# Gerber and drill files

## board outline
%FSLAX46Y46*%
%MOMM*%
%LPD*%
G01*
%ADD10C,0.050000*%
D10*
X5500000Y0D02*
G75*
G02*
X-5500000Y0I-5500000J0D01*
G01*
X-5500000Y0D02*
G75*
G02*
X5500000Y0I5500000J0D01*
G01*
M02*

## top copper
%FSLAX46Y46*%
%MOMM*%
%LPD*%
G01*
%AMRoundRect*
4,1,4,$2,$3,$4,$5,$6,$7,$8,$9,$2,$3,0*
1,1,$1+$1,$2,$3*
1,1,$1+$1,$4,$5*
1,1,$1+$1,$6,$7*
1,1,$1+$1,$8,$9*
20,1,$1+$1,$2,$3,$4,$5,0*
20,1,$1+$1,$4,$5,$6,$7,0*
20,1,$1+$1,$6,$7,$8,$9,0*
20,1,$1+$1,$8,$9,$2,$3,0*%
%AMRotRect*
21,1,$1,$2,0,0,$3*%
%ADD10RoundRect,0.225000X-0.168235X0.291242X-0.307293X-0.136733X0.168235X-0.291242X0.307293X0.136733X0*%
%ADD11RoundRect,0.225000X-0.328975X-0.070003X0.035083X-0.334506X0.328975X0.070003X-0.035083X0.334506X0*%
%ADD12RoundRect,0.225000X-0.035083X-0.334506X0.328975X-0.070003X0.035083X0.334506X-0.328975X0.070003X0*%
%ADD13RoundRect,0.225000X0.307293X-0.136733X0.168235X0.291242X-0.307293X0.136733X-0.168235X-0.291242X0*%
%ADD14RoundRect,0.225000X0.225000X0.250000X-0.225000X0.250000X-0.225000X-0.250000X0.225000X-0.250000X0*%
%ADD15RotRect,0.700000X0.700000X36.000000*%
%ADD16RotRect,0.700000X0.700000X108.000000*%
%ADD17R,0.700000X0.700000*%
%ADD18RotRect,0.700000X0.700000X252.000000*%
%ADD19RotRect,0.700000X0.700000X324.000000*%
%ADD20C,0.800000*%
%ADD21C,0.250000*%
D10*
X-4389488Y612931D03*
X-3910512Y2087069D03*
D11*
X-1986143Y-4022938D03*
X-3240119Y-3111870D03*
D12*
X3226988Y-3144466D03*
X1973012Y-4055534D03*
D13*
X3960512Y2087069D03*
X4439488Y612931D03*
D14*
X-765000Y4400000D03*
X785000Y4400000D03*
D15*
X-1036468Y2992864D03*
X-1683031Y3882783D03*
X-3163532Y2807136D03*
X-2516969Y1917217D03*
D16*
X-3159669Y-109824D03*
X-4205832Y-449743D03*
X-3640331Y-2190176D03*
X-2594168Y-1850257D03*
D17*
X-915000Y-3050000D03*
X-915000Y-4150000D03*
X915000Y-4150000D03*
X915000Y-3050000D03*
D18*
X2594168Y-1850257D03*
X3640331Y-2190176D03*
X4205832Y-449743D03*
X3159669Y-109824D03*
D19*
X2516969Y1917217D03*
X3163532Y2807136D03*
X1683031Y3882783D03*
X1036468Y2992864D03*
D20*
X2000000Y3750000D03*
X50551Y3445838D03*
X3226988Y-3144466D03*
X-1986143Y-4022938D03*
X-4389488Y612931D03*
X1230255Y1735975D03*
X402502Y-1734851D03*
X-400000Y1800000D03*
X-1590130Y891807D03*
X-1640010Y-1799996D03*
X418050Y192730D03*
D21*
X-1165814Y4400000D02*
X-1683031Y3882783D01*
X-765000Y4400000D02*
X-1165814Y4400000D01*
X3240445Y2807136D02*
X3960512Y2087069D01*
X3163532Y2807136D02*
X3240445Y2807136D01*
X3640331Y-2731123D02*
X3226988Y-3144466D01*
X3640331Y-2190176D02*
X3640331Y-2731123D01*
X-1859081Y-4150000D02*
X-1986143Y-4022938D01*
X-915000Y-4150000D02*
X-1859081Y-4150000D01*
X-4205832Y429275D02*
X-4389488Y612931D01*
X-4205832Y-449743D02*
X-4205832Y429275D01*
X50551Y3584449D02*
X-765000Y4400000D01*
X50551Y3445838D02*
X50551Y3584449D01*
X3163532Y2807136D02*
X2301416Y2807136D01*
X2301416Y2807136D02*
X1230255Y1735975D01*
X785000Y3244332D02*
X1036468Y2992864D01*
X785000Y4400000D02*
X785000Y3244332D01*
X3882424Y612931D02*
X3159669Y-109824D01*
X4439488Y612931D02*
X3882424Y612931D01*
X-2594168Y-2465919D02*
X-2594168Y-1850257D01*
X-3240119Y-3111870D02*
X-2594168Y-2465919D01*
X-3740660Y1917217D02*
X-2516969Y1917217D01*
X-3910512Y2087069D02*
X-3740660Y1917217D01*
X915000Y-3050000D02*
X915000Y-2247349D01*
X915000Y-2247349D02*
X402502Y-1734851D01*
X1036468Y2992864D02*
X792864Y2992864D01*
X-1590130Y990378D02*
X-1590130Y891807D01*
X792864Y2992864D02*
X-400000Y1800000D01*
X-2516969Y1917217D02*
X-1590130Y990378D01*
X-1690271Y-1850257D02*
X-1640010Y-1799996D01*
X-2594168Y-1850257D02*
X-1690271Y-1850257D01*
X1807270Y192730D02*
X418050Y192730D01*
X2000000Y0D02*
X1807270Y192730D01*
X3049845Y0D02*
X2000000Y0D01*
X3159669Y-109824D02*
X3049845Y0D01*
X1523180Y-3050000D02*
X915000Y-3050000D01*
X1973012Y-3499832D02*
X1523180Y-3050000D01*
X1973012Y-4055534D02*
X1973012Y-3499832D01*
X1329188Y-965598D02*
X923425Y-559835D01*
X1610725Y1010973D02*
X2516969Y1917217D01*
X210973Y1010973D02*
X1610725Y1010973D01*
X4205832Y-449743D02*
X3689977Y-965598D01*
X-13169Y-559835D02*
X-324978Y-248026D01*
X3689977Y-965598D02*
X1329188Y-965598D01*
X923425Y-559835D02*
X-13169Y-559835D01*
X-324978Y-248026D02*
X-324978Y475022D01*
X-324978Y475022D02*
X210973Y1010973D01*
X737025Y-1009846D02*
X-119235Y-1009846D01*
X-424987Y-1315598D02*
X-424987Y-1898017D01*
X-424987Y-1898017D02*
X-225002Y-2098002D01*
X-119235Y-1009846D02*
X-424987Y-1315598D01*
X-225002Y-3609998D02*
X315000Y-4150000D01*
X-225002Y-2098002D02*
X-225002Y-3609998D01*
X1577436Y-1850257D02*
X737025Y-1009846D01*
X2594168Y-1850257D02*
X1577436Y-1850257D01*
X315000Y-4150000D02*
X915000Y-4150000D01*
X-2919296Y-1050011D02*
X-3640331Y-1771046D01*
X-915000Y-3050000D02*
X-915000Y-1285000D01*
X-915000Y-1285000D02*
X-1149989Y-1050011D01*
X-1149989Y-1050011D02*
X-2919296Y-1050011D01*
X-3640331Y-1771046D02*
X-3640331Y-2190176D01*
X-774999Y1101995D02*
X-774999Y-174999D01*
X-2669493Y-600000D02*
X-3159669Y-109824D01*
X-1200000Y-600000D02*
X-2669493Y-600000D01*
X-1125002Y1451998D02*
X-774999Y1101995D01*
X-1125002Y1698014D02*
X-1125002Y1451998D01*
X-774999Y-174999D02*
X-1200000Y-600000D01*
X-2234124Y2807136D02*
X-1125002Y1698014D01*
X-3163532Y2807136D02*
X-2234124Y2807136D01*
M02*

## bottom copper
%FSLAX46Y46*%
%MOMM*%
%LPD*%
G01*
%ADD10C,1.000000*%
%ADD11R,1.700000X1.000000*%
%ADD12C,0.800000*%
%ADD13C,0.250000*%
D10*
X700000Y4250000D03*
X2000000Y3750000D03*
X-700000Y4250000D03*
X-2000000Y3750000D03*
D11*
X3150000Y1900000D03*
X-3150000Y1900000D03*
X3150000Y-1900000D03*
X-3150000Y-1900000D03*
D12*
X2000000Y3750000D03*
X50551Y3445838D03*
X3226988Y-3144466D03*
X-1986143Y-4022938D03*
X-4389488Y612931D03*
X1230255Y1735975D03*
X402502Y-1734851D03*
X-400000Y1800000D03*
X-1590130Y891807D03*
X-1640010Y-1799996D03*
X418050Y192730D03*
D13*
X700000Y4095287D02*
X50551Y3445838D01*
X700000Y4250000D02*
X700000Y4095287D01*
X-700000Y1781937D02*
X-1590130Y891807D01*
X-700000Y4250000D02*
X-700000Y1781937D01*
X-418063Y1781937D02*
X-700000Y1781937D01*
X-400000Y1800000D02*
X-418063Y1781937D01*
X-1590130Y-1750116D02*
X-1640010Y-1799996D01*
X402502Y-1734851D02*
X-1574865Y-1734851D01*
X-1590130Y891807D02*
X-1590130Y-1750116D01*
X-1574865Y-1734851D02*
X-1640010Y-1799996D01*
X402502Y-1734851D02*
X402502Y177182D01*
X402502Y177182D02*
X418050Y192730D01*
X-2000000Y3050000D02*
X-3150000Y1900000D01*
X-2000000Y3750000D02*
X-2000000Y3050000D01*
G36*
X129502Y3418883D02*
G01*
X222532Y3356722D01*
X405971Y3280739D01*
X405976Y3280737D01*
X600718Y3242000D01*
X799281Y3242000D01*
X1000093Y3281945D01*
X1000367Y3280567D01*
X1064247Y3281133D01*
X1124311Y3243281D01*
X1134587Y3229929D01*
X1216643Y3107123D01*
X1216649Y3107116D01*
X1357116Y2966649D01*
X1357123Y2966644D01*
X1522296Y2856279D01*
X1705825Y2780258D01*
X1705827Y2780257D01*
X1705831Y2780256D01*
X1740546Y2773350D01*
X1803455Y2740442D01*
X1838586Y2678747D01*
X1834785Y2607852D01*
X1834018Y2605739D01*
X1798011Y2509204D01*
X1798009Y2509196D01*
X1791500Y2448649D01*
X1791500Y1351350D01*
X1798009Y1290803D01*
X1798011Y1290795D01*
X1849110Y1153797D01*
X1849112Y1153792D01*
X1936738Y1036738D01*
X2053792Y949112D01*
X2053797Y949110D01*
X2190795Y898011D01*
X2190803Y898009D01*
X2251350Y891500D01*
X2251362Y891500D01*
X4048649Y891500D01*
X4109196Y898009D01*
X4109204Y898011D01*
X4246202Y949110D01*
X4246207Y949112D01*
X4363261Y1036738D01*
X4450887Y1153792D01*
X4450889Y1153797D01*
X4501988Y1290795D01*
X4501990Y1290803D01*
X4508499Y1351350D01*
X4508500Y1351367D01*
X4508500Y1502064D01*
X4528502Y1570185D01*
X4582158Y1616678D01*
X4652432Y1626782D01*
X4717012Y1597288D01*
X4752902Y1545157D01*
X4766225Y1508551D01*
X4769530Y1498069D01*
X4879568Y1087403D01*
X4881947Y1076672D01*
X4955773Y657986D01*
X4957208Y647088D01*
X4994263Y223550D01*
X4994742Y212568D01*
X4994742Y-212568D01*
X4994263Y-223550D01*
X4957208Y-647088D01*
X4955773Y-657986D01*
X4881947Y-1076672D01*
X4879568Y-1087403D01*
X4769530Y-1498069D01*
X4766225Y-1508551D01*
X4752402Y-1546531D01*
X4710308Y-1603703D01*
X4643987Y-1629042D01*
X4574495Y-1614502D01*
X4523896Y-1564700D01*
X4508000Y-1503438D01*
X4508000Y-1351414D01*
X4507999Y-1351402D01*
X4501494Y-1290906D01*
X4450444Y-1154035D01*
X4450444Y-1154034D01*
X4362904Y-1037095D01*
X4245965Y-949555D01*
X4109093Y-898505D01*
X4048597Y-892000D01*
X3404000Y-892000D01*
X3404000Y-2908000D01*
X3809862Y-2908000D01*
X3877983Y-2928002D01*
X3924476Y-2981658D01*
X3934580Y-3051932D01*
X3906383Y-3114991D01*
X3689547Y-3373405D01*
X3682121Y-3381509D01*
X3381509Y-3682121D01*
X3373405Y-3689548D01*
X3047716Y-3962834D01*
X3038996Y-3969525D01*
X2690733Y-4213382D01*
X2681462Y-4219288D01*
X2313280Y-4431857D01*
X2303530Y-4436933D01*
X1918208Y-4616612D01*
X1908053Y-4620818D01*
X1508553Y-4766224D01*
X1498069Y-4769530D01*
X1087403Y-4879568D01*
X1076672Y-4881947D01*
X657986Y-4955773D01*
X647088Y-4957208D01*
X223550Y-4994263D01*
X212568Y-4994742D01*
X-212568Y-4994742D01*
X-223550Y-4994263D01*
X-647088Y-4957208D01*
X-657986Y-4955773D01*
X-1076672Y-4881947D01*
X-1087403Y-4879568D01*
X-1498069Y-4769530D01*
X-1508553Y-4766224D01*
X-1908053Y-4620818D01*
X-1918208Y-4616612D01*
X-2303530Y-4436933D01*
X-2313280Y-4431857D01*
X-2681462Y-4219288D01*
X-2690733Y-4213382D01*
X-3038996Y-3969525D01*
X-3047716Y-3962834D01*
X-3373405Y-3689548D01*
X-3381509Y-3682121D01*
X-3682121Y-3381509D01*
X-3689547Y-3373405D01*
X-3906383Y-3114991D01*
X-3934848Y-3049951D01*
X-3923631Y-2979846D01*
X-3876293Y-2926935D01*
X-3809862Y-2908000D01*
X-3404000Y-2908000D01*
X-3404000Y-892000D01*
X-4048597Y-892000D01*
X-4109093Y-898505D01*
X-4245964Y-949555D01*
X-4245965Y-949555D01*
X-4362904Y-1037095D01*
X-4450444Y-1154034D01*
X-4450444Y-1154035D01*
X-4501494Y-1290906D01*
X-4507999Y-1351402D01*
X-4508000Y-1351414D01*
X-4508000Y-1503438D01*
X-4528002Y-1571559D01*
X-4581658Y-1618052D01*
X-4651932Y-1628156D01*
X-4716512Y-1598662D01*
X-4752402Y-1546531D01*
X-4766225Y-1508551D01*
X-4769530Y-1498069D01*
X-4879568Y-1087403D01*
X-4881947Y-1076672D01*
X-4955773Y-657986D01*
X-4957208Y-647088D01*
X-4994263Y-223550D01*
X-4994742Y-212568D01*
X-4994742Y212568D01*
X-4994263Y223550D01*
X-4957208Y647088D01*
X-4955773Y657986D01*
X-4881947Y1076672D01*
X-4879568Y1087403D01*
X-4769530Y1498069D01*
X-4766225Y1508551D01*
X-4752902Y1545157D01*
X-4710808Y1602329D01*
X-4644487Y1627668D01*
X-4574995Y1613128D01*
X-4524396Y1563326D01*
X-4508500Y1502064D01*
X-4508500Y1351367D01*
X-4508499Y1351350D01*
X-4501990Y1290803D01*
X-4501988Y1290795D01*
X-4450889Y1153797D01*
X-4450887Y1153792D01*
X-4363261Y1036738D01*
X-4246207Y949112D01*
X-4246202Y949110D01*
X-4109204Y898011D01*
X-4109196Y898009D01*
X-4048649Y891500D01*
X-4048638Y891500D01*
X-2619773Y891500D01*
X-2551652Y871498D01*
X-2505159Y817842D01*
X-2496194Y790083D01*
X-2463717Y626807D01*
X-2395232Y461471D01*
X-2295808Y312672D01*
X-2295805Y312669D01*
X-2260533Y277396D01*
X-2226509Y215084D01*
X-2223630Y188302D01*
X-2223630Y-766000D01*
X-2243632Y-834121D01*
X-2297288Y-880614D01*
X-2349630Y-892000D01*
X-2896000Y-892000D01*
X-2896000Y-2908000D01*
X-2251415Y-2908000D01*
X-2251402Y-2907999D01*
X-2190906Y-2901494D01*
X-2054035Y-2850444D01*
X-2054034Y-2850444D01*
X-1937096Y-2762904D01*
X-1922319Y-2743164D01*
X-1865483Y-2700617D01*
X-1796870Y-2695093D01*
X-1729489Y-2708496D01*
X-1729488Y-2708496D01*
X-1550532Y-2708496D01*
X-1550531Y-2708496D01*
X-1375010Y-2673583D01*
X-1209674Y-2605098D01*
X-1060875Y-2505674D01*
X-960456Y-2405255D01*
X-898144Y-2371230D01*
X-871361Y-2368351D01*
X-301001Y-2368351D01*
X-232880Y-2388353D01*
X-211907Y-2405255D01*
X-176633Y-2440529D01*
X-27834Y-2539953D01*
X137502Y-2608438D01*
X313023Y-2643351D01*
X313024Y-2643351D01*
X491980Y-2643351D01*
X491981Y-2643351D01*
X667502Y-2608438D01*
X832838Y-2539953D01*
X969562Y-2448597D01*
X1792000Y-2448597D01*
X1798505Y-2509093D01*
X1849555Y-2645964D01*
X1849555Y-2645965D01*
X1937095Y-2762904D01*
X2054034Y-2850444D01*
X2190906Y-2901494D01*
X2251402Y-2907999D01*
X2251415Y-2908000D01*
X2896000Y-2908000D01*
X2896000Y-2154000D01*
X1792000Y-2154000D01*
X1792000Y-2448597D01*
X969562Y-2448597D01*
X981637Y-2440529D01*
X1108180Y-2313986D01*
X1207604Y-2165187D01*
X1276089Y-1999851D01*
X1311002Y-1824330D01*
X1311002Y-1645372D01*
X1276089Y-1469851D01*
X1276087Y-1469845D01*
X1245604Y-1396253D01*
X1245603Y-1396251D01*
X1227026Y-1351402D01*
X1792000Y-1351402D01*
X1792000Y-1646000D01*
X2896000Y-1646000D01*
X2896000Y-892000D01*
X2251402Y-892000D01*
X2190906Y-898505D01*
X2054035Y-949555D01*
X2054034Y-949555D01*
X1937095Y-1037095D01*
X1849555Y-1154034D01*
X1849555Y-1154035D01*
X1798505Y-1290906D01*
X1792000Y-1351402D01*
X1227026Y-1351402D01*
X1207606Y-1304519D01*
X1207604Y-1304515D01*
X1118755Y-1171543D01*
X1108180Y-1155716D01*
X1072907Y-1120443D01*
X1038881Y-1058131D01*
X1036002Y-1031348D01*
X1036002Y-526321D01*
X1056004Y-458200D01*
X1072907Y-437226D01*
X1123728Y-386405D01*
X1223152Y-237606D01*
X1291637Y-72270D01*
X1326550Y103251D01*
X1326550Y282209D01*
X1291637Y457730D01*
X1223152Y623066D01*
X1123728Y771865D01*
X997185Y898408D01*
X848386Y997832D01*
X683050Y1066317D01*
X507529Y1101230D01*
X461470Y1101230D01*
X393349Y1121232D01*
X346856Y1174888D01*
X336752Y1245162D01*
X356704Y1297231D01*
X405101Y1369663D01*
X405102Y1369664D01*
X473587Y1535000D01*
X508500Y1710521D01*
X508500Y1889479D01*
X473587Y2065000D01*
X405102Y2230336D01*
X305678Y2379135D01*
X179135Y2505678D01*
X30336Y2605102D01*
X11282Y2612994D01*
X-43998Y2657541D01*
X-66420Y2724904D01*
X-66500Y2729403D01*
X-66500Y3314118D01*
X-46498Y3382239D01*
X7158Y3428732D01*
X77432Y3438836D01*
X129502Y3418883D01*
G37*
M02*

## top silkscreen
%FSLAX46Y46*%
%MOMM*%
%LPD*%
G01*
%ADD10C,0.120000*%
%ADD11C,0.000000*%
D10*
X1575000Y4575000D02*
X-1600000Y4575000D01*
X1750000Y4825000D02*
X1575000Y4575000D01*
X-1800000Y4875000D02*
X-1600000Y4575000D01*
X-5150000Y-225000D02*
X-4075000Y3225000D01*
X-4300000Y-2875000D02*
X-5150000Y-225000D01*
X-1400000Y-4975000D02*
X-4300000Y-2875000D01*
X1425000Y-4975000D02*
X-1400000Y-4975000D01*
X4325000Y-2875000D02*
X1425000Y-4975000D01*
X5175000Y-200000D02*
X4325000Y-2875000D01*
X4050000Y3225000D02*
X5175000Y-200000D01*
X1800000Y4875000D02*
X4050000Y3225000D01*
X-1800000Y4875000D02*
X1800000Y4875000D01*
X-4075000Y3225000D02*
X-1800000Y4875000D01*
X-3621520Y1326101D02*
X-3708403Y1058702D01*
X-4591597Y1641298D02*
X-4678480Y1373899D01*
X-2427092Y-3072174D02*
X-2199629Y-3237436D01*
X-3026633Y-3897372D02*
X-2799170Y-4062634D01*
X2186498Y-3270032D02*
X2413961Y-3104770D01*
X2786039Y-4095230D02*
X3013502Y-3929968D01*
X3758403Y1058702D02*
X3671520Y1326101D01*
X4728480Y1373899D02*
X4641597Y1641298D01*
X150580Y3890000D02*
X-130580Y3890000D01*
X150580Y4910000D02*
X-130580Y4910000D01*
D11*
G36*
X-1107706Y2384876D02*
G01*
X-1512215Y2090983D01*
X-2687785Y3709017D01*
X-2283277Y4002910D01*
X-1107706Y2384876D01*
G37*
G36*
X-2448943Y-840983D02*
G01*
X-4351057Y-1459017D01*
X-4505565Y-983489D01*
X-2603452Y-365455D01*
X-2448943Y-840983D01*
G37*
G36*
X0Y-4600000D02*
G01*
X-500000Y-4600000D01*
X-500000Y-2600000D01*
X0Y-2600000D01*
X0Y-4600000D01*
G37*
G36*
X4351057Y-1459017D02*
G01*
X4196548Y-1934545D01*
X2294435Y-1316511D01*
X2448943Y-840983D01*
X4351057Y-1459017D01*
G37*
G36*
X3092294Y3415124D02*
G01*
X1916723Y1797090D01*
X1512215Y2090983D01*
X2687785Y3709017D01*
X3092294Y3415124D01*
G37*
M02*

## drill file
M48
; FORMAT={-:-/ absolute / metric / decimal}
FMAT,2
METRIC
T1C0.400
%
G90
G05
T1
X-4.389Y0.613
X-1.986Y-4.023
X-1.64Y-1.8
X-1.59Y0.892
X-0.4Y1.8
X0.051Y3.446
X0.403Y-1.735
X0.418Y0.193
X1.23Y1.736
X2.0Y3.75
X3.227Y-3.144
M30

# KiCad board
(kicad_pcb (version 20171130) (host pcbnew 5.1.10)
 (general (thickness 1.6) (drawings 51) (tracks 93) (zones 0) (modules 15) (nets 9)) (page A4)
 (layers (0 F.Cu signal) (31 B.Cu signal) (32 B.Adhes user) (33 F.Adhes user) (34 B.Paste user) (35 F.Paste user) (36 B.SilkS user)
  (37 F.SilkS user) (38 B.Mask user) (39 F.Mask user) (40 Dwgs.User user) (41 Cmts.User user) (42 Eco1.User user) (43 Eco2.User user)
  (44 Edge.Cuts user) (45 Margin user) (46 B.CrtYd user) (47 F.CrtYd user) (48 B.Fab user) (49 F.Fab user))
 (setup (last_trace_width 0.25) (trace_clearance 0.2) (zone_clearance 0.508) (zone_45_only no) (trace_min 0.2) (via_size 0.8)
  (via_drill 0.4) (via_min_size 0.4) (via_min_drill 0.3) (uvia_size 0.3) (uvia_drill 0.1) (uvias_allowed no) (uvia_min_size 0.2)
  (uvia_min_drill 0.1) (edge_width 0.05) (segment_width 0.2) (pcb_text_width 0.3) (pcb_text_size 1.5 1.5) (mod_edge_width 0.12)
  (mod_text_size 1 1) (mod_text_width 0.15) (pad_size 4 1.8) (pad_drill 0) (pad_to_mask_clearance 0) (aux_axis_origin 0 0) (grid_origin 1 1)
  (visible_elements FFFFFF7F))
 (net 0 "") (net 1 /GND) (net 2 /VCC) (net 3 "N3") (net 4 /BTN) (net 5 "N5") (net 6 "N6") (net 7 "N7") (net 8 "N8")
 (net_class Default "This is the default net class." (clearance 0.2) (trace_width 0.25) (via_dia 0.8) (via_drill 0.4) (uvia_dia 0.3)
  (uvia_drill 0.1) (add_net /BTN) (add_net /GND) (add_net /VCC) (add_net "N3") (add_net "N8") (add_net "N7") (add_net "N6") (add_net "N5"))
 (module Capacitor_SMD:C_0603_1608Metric (layer F.Cu) (at -4.15 -1.35 252)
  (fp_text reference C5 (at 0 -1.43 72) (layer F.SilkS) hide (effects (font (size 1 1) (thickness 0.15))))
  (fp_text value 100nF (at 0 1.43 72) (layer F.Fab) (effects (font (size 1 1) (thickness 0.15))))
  (fp_line (start -0.14058 -0.51) (end 0.14058 -0.51) (layer F.SilkS) (width 0.12))
  (fp_line (start -0.14058 0.51) (end 0.14058 0.51) (layer F.SilkS) (width 0.12))
  (pad 2 smd roundrect (at 0.775 0 252) (size 0.9 0.95) (layers F.Cu F.Paste F.Mask) (roundrect_rratio 0.25) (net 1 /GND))
  (pad 1 smd roundrect (at -0.775 0 252) (size 0.9 0.95) (layers F.Cu F.Paste F.Mask) (roundrect_rratio 0.25) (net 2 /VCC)))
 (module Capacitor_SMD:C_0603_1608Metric (layer F.Cu) (at -2.613131 3.567404 324)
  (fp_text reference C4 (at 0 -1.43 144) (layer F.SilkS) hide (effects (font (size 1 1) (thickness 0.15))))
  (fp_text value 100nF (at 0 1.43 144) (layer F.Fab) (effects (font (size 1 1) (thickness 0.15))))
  (fp_line (start -0.14058 -0.51) (end 0.14058 -0.51) (layer F.SilkS) (width 0.12))
  (fp_line (start -0.14058 0.51) (end 0.14058 0.51) (layer F.SilkS) (width 0.12))
  (pad 2 smd roundrect (at 0.775 0 324) (size 0.9 0.95) (layers F.Cu F.Paste F.Mask) (roundrect_rratio 0.25) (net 1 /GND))
  (pad 1 smd roundrect (at -0.775 0 324) (size 0.9 0.95) (layers F.Cu F.Paste F.Mask) (roundrect_rratio 0.25) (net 2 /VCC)))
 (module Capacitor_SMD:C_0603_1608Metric (layer F.Cu) (at 2.6 3.6 36)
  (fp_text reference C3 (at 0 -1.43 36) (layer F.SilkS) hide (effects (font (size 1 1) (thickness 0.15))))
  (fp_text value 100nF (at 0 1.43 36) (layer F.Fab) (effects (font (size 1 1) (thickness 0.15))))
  (fp_line (start -0.14058 -0.51) (end 0.14058 -0.51) (layer F.SilkS) (width 0.12))
  (fp_line (start -0.14058 0.51) (end 0.14058 0.51) (layer F.SilkS) (width 0.12))
  (pad 2 smd roundrect (at 0.775 0 36) (size 0.9 0.95) (layers F.Cu F.Paste F.Mask) (roundrect_rratio 0.25) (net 1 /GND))
  (pad 1 smd roundrect (at -0.775 0 36) (size 0.9 0.95) (layers F.Cu F.Paste F.Mask) (roundrect_rratio 0.25) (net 2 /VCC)))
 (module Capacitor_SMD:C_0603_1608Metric (layer F.Cu) (at 4.2 -1.35 108)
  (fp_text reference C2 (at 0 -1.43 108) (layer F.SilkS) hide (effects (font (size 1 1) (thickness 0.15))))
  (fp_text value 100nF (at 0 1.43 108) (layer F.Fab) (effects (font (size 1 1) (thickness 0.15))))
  (fp_line (start -0.14058 -0.51) (end 0.14058 -0.51) (layer F.SilkS) (width 0.12))
  (fp_line (start -0.14058 0.51) (end 0.14058 0.51) (layer F.SilkS) (width 0.12))
  (pad 2 smd roundrect (at 0.775 0 108) (size 0.9 0.95) (layers F.Cu F.Paste F.Mask) (roundrect_rratio 0.25) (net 1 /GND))
  (pad 1 smd roundrect (at -0.775 0 108) (size 0.9 0.95) (layers F.Cu F.Paste F.Mask) (roundrect_rratio 0.25) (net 2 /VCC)))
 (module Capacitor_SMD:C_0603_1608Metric (layer F.Cu) (at 0.01 -4.4 180)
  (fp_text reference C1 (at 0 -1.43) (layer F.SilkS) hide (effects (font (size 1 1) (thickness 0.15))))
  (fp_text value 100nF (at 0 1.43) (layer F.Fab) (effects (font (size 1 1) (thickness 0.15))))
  (fp_line (start -0.14058 -0.51) (end 0.14058 -0.51) (layer F.SilkS) (width 0.12))
  (fp_line (start -0.14058 0.51) (end 0.14058 0.51) (layer F.SilkS) (width 0.12))
  (pad 2 smd roundrect (at 0.775 0 180) (size 0.9 0.95) (layers F.Cu F.Paste F.Mask) (roundrect_rratio 0.25) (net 1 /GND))
  (pad 1 smd roundrect (at -0.775 0 180) (size 0.9 0.95) (layers F.Cu F.Paste F.Mask) (roundrect_rratio 0.25) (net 2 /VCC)))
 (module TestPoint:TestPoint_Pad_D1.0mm (layer B.Cu) (at 0.7 -4.25)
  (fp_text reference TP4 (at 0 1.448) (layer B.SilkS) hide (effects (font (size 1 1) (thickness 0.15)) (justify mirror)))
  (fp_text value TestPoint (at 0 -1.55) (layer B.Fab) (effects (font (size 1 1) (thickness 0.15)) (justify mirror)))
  (pad 1 smd circle (at 0 0) (size 1 1) (layers B.Cu B.Mask) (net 1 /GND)))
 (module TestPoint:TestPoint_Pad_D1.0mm (layer B.Cu) (at 2 -3.75)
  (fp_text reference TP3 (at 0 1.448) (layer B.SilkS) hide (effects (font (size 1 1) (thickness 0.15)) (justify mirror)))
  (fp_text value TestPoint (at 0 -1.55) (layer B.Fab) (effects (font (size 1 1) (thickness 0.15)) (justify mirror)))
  (pad 1 smd circle (at 0 0) (size 1 1) (layers B.Cu B.Mask) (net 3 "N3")))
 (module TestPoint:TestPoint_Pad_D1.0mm (layer B.Cu) (at -0.7 -4.25)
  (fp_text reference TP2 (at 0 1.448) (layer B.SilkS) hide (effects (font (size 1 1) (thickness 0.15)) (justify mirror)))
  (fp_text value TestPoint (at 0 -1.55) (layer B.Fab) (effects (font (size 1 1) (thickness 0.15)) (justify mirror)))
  (pad 1 smd circle (at 0 0) (size 1 1) (layers B.Cu B.Mask) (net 2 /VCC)))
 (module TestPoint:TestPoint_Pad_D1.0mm (layer B.Cu) (at -2 -3.75)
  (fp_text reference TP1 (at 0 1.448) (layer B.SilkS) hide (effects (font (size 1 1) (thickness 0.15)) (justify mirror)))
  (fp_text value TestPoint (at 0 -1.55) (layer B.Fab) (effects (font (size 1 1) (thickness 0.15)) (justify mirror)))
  (pad 1 smd circle (at 0 0) (size 1 1) (layers B.Cu B.Mask) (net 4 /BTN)))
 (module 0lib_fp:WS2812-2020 (layer F.Cu) (at -2.1 -2.9 36)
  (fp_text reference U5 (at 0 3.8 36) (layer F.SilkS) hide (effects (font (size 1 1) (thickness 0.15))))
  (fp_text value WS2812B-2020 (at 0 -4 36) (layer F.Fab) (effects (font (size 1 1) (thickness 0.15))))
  (fp_poly (pts (xy 0 -1) (xy 0.5 -1) (xy 0.5 1) (xy 0 1)) (layer F.SilkS) (width 0))
  (pad 1 smd rect (at 0.915 0.55 36) (size 0.7 0.7) (layers F.Cu F.Paste F.Mask))
  (pad 2 smd rect (at 0.915 -0.55 36) (size 0.7 0.7) (layers F.Cu F.Paste F.Mask) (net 1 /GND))
  (pad 3 smd rect (at -0.915 -0.55 36) (size 0.7 0.7) (layers F.Cu F.Paste F.Mask) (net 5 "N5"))
  (pad 4 smd rect (at -0.915 0.55 36) (size 0.7 0.7) (layers F.Cu F.Paste F.Mask) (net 2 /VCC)))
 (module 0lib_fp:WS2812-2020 (layer F.Cu) (at -3.4 1.15 108)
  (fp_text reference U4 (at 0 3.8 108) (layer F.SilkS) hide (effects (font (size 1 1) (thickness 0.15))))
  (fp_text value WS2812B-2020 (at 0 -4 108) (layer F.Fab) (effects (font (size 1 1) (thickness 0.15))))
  (fp_poly (pts (xy 0 -1) (xy 0.5 -1) (xy 0.5 1) (xy 0 1)) (layer F.SilkS) (width 0))
  (pad 1 smd rect (at 0.915 0.55 108) (size 0.7 0.7) (layers F.Cu F.Paste F.Mask) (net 5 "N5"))
  (pad 2 smd rect (at 0.915 -0.55 108) (size 0.7 0.7) (layers F.Cu F.Paste F.Mask) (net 1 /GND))
  (pad 3 smd rect (at -0.915 -0.55 108) (size 0.7 0.7) (layers F.Cu F.Paste F.Mask) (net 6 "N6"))
  (pad 4 smd rect (at -0.915 0.55 108) (size 0.7 0.7) (layers F.Cu F.Paste F.Mask) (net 2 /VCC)))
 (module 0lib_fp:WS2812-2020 (layer F.Cu) (at 0 3.6 180)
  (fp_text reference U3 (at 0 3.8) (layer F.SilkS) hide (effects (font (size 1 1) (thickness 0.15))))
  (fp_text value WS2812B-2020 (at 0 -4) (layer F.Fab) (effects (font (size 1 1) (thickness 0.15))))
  (fp_poly (pts (xy 0 -1) (xy 0.5 -1) (xy 0.5 1) (xy 0 1)) (layer F.SilkS) (width 0))
  (pad 1 smd rect (at 0.915 0.55 180) (size 0.7 0.7) (layers F.Cu F.Paste F.Mask) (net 6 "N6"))
  (pad 2 smd rect (at 0.915 -0.55 180) (size 0.7 0.7) (layers F.Cu F.Paste F.Mask) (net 1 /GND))
  (pad 3 smd rect (at -0.915 -0.55 180) (size 0.7 0.7) (layers F.Cu F.Paste F.Mask) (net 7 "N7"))
  (pad 4 smd rect (at -0.915 0.55 180) (size 0.7 0.7) (layers F.Cu F.Paste F.Mask) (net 2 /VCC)))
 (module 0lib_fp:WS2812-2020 (layer F.Cu) (at 3.4 1.15 252)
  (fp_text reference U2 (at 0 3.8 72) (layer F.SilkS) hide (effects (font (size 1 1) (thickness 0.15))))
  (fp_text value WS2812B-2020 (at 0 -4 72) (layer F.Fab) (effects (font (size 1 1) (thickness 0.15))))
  (fp_poly (pts (xy 0 -1) (xy 0.5 -1) (xy 0.5 1) (xy 0 1)) (layer F.SilkS) (width 0))
  (pad 1 smd rect (at 0.915 0.55 252) (size 0.7 0.7) (layers F.Cu F.Paste F.Mask) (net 7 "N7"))
  (pad 2 smd rect (at 0.915 -0.55 252) (size 0.7 0.7) (layers F.Cu F.Paste F.Mask) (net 1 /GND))
  (pad 3 smd rect (at -0.915 -0.55 252) (size 0.7 0.7) (layers F.Cu F.Paste F.Mask) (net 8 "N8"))
  (pad 4 smd rect (at -0.915 0.55 252) (size 0.7 0.7) (layers F.Cu F.Paste F.Mask) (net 2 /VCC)))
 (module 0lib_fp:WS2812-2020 (layer F.Cu) (at 2.1 -2.9 324)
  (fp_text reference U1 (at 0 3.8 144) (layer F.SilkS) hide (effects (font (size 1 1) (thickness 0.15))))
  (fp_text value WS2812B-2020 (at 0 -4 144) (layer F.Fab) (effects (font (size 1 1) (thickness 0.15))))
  (fp_poly (pts (xy 0 -1) (xy 0.5 -1) (xy 0.5 1) (xy 0 1)) (layer F.SilkS) (width 0))
  (pad 1 smd rect (at 0.915 0.55 324) (size 0.7 0.7) (layers F.Cu F.Paste F.Mask) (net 8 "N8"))
  (pad 2 smd rect (at 0.915 -0.55 324) (size 0.7 0.7) (layers F.Cu F.Paste F.Mask) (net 1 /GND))
  (pad 3 smd rect (at -0.915 -0.55 324) (size 0.7 0.7) (layers F.Cu F.Paste F.Mask) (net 3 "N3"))
  (pad 4 smd rect (at -0.915 0.55 324) (size 0.7 0.7) (layers F.Cu F.Paste F.Mask) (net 2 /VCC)))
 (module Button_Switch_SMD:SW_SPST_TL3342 (layer B.Cu) (at 0 0)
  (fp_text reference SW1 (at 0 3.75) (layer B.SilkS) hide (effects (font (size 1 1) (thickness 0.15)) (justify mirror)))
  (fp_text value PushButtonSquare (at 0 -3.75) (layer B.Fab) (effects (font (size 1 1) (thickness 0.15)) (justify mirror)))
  (pad 2 smd rect (at 3.15 -1.9) (size 1.7 1) (layers B.Cu B.Paste B.Mask) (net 4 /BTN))
  (pad 2 smd rect (at -3.15 -1.9) (size 1.7 1) (layers B.Cu B.Paste B.Mask) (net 4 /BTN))
  (pad 1 smd rect (at 3.15 1.9) (size 1.7 1) (layers B.Cu B.Paste B.Mask) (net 1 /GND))
  (pad 1 smd rect (at -3.15 1.9) (size 1.7 1) (layers B.Cu B.Paste B.Mask) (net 1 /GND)))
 (gr_line (start 1.575 -4.575) (end -1.6 -4.575) (layer F.SilkS) (width 0.12))
 (gr_line (start 1.75 -4.825) (end 1.575 -4.575) (layer F.SilkS) (width 0.12))
 (gr_line (start -1.8 -4.875) (end -1.6 -4.575) (layer F.SilkS) (width 0.12))
 (gr_line (start -5.15 0.225) (end -4.075 -3.225) (layer F.SilkS) (width 0.12))
 (gr_line (start -4.3 2.875) (end -5.15 0.225) (layer F.SilkS) (width 0.12))
 (gr_line (start -1.4 4.975) (end -4.3 2.875) (layer F.SilkS) (width 0.12))
 (gr_line (start 1.425 4.975) (end -1.4 4.975) (layer F.SilkS) (width 0.12))
 (gr_line (start 4.325 2.875) (end 1.425 4.975) (layer F.SilkS) (width 0.12))
 (gr_line (start 5.175 0.2) (end 4.325 2.875) (layer F.SilkS) (width 0.12))
 (gr_line (start 4.05 -3.225) (end 5.175 0.2) (layer F.SilkS) (width 0.12))
 (gr_line (start 1.8 -4.875) (end 4.05 -3.225) (layer F.SilkS) (width 0.12))
 (gr_line (start -1.8 -4.875) (end 1.8 -4.875) (layer F.SilkS) (width 0.12))
 (gr_line (start -4.075 -3.225) (end -1.8 -4.875) (layer F.SilkS) (width 0.12))
 (gr_circle (center 0 0) (end 0 -5.5) (layer Edge.Cuts) (width 0.05))
 (via (at 2 -3.75) (size 0.8) (drill 0.4) (layers F.Cu B.Cu) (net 3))
 (segment (start -1.165814 -4.4) (end -1.683031 -3.882783) (width 0.25) (layer F.Cu) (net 1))
 (segment (start -0.765 -4.4) (end -1.165814 -4.4) (width 0.25) (layer F.Cu) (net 1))
 (segment (start 3.240445 -2.807136) (end 3.960512 -2.087069) (width 0.25) (layer F.Cu) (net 1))
 (segment (start 3.163532 -2.807136) (end 3.240445 -2.807136) (width 0.25) (layer F.Cu) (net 1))
 (segment (start 3.640331 2.731123) (end 3.226988 3.144466) (width 0.25) (layer F.Cu) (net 1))
 (segment (start 3.640331 2.190176) (end 3.640331 2.731123) (width 0.25) (layer F.Cu) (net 1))
 (segment (start -1.859081 4.15) (end -1.986143 4.022938) (width 0.25) (layer F.Cu) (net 1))
 (segment (start -0.915 4.15) (end -1.859081 4.15) (width 0.25) (layer F.Cu) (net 1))
 (segment (start -4.205832 -0.429275) (end -4.389488 -0.612931) (width 0.25) (layer F.Cu) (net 1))
 (segment (start -4.205832 0.449743) (end -4.205832 -0.429275) (width 0.25) (layer F.Cu) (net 1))
 (via (at 0.050551 -3.445838) (size 0.8) (drill 0.4) (layers F.Cu B.Cu) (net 1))
 (segment (start 0.7 -4.095287) (end 0.050551 -3.445838) (width 0.25) (layer B.Cu) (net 1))
 (segment (start 0.7 -4.25) (end 0.7 -4.095287) (width 0.25) (layer B.Cu) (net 1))
 (segment (start 0.050551 -3.584449) (end -0.765 -4.4) (width 0.25) (layer F.Cu) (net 1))
 (segment (start 0.050551 -3.445838) (end 0.050551 -3.584449) (width 0.25) (layer F.Cu) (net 1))
 (via (at 3.226988 3.144466) (size 0.8) (drill 0.4) (layers F.Cu B.Cu) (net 1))
 (via (at -1.986143 4.022938) (size 0.8) (drill 0.4) (layers F.Cu B.Cu) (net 1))
 (via (at -4.389488 -0.612931) (size 0.8) (drill 0.4) (layers F.Cu B.Cu) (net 1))
 (segment (start 3.163532 -2.807136) (end 2.301416 -2.807136) (width 0.25) (layer F.Cu) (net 1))
 (segment (start 2.301416 -2.807136) (end 1.230255 -1.735975) (width 0.25) (layer F.Cu) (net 1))
 (via (at 1.230255 -1.735975) (size 0.8) (drill 0.4) (layers F.Cu B.Cu) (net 1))
 (segment (start 0.785 -3.244332) (end 1.036468 -2.992864) (width 0.25) (layer F.Cu) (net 2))
 (segment (start 0.785 -4.4) (end 0.785 -3.244332) (width 0.25) (layer F.Cu) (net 2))
 (segment (start 3.882424 -0.612931) (end 3.159669 0.109824) (width 0.25) (layer F.Cu) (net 2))
 (segment (start 4.439488 -0.612931) (end 3.882424 -0.612931) (width 0.25) (layer F.Cu) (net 2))
 (segment (start -2.594168 2.465919) (end -2.594168 1.850257) (width 0.25) (layer F.Cu) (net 2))
 (segment (start -3.240119 3.11187) (end -2.594168 2.465919) (width 0.25) (layer F.Cu) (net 2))
 (segment (start -3.74066 -1.917217) (end -2.516969 -1.917217) (width 0.25) (layer F.Cu) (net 2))
 (segment (start -3.910512 -2.087069) (end -3.74066 -1.917217) (width 0.25) (layer F.Cu) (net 2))
 (segment (start 0.915 3.05) (end 0.915 2.247349) (width 0.25) (layer F.Cu) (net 2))
 (via (at 0.402502 1.734851) (size 0.8) (drill 0.4) (layers F.Cu B.Cu) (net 2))
 (segment (start 0.915 2.247349) (end 0.402502 1.734851) (width 0.25) (layer F.Cu) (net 2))
 (via (at -0.4 -1.8) (size 0.8) (drill 0.4) (layers F.Cu B.Cu) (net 2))
 (segment (start 1.036468 -2.992864) (end 0.792864 -2.992864) (width 0.25) (layer F.Cu) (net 2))
 (via (at -1.59013 -0.891807) (size 0.8) (drill 0.4) (layers F.Cu B.Cu) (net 2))
 (segment (start -1.59013 -0.990378) (end -1.59013 -0.891807) (width 0.25) (layer F.Cu) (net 2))
 (segment (start -0.7 -1.781937) (end -1.59013 -0.891807) (width 0.25) (layer B.Cu) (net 2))
 (segment (start 0.792864 -2.992864) (end -0.4 -1.8) (width 0.25) (layer F.Cu) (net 2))
 (segment (start -0.7 -4.25) (end -0.7 -1.781937) (width 0.25) (layer B.Cu) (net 2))
 (segment (start -2.516969 -1.917217) (end -1.59013 -0.990378) (width 0.25) (layer F.Cu) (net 2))
 (segment (start -0.418063 -1.781937) (end -0.7 -1.781937) (width 0.25) (layer B.Cu) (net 2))
 (segment (start -0.4 -1.8) (end -0.418063 -1.781937) (width 0.25) (layer B.Cu) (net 2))
 (segment (start -1.690271 1.850257) (end -1.64001 1.799996) (width 0.25) (layer F.Cu) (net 2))
 (segment (start -1.59013 1.750116) (end -1.64001 1.799996) (width 0.25) (layer B.Cu) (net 2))
 (segment (start 0.402502 1.734851) (end -1.574865 1.734851) (width 0.25) (layer B.Cu) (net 2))
 (via (at -1.64001 1.799996) (size 0.8) (drill 0.4) (layers F.Cu B.Cu) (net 2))
 (segment (start -2.594168 1.850257) (end -1.690271 1.850257) (width 0.25) (layer F.Cu) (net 2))
 (segment (start -1.59013 -0.891807) (end -1.59013 1.750116) (width 0.25) (layer B.Cu) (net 2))
 (segment (start -1.574865 1.734851) (end -1.64001 1.799996) (width 0.25) (layer B.Cu) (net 2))
 (segment (start 0.402502 1.734851) (end 0.402502 -0.177182) (width 0.25) (layer B.Cu) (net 2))
 (segment (start 0.402502 -0.177182) (end 0.41805 -0.19273) (width 0.25) (layer B.Cu) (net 2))
 (via (at 0.41805 -0.19273) (size 0.8) (drill 0.4) (layers F.Cu B.Cu) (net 2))
 (segment (start 1.80727 -0.19273) (end 0.41805 -0.19273) (width 0.25) (layer F.Cu) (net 2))
 (segment (start 2 0) (end 1.80727 -0.19273) (width 0.25) (layer F.Cu) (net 2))
 (segment (start 3.049845 0) (end 2 0) (width 0.25) (layer F.Cu) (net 2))
 (segment (start 3.159669 0.109824) (end 3.049845 0) (width 0.25) (layer F.Cu) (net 2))
 (segment (start 1.52318 3.05) (end 0.915 3.05) (width 0.25) (layer F.Cu) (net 2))
 (segment (start 1.973012 3.499832) (end 1.52318 3.05) (width 0.25) (layer F.Cu) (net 2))
 (segment (start 1.973012 4.055534) (end 1.973012 3.499832) (width 0.25) (layer F.Cu) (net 2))
 (segment (start -2 -3.05) (end -3.15 -1.9) (width 0.25) (layer B.Cu) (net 4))
 (segment (start -2 -3.75) (end -2 -3.05) (width 0.25) (layer B.Cu) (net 4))
 (segment (start 1.329188 0.965598) (end 0.923425 0.559835) (width 0.25) (layer F.Cu) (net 8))
 (segment (start 1.610725 -1.010973) (end 2.516969 -1.917217) (width 0.25) (layer F.Cu) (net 8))
 (segment (start 0.210973 -1.010973) (end 1.610725 -1.010973) (width 0.25) (layer F.Cu) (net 8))
 (segment (start 4.205832 0.449743) (end 3.689977 0.965598) (width 0.25) (layer F.Cu) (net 8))
 (segment (start -0.013169 0.559835) (end -0.324978 0.248026) (width 0.25) (layer F.Cu) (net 8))
 (segment (start 3.689977 0.965598) (end 1.329188 0.965598) (width 0.25) (layer F.Cu) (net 8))
 (segment (start 0.923425 0.559835) (end -0.013169 0.559835) (width 0.25) (layer F.Cu) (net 8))
 (segment (start -0.324978 0.248026) (end -0.324978 -0.475022) (width 0.25) (layer F.Cu) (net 8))
 (segment (start -0.324978 -0.475022) (end 0.210973 -1.010973) (width 0.25) (layer F.Cu) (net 8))
 (segment (start 0.737025 1.009846) (end -0.119235 1.009846) (width 0.25) (layer F.Cu) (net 7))
 (segment (start -0.424987 1.315598) (end -0.424987 1.898017) (width 0.25) (layer F.Cu) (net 7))
 (segment (start -0.424987 1.898017) (end -0.225002 2.098002) (width 0.25) (layer F.Cu) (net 7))
 (segment (start -0.119235 1.009846) (end -0.424987 1.315598) (width 0.25) (layer F.Cu) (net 7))
 (segment (start -0.225002 3.609998) (end 0.315 4.15) (width 0.25) (layer F.Cu) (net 7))
 (segment (start -0.225002 2.098002) (end -0.225002 3.609998) (width 0.25) (layer F.Cu) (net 7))
 (segment (start 1.577436 1.850257) (end 0.737025 1.009846) (width 0.25) (layer F.Cu) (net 7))
 (segment (start 2.594168 1.850257) (end 1.577436 1.850257) (width 0.25) (layer F.Cu) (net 7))
 (segment (start 0.315 4.15) (end 0.915 4.15) (width 0.25) (layer F.Cu) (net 7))
 (segment (start -2.919296 1.050011) (end -3.640331 1.771046) (width 0.25) (layer F.Cu) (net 6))
 (segment (start -0.915 3.05) (end -0.915 1.285) (width 0.25) (layer F.Cu) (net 6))
 (segment (start -0.915 1.285) (end -1.149989 1.050011) (width 0.25) (layer F.Cu) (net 6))
 (segment (start -1.149989 1.050011) (end -2.919296 1.050011) (width 0.25) (layer F.Cu) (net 6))
 (segment (start -3.640331 1.771046) (end -3.640331 2.190176) (width 0.25) (layer F.Cu) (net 6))
 (segment (start -0.774999 -1.101995) (end -0.774999 0.174999) (width 0.25) (layer F.Cu) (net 5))
 (segment (start -2.669493 0.6) (end -3.159669 0.109824) (width 0.25) (layer F.Cu) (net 5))
 (segment (start -1.2 0.6) (end -2.669493 0.6) (width 0.25) (layer F.Cu) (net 5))
 (segment (start -1.125002 -1.451998) (end -0.774999 -1.101995) (width 0.25) (layer F.Cu) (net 5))
 (segment (start -1.125002 -1.698014) (end -1.125002 -1.451998) (width 0.25) (layer F.Cu) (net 5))
 (segment (start -0.774999 0.174999) (end -1.2 0.6) (width 0.25) (layer F.Cu) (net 5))
 (segment (start -2.234124 -2.807136) (end -1.125002 -1.698014) (width 0.25) (layer F.Cu) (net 5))
 (segment (start -3.163532 -2.807136) (end -2.234124 -2.807136) (width 0.25) (layer F.Cu) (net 5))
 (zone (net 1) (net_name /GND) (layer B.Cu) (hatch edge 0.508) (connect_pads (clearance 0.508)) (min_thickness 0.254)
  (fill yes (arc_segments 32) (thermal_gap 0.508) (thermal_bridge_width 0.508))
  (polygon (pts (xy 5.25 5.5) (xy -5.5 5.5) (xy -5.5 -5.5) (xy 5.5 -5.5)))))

